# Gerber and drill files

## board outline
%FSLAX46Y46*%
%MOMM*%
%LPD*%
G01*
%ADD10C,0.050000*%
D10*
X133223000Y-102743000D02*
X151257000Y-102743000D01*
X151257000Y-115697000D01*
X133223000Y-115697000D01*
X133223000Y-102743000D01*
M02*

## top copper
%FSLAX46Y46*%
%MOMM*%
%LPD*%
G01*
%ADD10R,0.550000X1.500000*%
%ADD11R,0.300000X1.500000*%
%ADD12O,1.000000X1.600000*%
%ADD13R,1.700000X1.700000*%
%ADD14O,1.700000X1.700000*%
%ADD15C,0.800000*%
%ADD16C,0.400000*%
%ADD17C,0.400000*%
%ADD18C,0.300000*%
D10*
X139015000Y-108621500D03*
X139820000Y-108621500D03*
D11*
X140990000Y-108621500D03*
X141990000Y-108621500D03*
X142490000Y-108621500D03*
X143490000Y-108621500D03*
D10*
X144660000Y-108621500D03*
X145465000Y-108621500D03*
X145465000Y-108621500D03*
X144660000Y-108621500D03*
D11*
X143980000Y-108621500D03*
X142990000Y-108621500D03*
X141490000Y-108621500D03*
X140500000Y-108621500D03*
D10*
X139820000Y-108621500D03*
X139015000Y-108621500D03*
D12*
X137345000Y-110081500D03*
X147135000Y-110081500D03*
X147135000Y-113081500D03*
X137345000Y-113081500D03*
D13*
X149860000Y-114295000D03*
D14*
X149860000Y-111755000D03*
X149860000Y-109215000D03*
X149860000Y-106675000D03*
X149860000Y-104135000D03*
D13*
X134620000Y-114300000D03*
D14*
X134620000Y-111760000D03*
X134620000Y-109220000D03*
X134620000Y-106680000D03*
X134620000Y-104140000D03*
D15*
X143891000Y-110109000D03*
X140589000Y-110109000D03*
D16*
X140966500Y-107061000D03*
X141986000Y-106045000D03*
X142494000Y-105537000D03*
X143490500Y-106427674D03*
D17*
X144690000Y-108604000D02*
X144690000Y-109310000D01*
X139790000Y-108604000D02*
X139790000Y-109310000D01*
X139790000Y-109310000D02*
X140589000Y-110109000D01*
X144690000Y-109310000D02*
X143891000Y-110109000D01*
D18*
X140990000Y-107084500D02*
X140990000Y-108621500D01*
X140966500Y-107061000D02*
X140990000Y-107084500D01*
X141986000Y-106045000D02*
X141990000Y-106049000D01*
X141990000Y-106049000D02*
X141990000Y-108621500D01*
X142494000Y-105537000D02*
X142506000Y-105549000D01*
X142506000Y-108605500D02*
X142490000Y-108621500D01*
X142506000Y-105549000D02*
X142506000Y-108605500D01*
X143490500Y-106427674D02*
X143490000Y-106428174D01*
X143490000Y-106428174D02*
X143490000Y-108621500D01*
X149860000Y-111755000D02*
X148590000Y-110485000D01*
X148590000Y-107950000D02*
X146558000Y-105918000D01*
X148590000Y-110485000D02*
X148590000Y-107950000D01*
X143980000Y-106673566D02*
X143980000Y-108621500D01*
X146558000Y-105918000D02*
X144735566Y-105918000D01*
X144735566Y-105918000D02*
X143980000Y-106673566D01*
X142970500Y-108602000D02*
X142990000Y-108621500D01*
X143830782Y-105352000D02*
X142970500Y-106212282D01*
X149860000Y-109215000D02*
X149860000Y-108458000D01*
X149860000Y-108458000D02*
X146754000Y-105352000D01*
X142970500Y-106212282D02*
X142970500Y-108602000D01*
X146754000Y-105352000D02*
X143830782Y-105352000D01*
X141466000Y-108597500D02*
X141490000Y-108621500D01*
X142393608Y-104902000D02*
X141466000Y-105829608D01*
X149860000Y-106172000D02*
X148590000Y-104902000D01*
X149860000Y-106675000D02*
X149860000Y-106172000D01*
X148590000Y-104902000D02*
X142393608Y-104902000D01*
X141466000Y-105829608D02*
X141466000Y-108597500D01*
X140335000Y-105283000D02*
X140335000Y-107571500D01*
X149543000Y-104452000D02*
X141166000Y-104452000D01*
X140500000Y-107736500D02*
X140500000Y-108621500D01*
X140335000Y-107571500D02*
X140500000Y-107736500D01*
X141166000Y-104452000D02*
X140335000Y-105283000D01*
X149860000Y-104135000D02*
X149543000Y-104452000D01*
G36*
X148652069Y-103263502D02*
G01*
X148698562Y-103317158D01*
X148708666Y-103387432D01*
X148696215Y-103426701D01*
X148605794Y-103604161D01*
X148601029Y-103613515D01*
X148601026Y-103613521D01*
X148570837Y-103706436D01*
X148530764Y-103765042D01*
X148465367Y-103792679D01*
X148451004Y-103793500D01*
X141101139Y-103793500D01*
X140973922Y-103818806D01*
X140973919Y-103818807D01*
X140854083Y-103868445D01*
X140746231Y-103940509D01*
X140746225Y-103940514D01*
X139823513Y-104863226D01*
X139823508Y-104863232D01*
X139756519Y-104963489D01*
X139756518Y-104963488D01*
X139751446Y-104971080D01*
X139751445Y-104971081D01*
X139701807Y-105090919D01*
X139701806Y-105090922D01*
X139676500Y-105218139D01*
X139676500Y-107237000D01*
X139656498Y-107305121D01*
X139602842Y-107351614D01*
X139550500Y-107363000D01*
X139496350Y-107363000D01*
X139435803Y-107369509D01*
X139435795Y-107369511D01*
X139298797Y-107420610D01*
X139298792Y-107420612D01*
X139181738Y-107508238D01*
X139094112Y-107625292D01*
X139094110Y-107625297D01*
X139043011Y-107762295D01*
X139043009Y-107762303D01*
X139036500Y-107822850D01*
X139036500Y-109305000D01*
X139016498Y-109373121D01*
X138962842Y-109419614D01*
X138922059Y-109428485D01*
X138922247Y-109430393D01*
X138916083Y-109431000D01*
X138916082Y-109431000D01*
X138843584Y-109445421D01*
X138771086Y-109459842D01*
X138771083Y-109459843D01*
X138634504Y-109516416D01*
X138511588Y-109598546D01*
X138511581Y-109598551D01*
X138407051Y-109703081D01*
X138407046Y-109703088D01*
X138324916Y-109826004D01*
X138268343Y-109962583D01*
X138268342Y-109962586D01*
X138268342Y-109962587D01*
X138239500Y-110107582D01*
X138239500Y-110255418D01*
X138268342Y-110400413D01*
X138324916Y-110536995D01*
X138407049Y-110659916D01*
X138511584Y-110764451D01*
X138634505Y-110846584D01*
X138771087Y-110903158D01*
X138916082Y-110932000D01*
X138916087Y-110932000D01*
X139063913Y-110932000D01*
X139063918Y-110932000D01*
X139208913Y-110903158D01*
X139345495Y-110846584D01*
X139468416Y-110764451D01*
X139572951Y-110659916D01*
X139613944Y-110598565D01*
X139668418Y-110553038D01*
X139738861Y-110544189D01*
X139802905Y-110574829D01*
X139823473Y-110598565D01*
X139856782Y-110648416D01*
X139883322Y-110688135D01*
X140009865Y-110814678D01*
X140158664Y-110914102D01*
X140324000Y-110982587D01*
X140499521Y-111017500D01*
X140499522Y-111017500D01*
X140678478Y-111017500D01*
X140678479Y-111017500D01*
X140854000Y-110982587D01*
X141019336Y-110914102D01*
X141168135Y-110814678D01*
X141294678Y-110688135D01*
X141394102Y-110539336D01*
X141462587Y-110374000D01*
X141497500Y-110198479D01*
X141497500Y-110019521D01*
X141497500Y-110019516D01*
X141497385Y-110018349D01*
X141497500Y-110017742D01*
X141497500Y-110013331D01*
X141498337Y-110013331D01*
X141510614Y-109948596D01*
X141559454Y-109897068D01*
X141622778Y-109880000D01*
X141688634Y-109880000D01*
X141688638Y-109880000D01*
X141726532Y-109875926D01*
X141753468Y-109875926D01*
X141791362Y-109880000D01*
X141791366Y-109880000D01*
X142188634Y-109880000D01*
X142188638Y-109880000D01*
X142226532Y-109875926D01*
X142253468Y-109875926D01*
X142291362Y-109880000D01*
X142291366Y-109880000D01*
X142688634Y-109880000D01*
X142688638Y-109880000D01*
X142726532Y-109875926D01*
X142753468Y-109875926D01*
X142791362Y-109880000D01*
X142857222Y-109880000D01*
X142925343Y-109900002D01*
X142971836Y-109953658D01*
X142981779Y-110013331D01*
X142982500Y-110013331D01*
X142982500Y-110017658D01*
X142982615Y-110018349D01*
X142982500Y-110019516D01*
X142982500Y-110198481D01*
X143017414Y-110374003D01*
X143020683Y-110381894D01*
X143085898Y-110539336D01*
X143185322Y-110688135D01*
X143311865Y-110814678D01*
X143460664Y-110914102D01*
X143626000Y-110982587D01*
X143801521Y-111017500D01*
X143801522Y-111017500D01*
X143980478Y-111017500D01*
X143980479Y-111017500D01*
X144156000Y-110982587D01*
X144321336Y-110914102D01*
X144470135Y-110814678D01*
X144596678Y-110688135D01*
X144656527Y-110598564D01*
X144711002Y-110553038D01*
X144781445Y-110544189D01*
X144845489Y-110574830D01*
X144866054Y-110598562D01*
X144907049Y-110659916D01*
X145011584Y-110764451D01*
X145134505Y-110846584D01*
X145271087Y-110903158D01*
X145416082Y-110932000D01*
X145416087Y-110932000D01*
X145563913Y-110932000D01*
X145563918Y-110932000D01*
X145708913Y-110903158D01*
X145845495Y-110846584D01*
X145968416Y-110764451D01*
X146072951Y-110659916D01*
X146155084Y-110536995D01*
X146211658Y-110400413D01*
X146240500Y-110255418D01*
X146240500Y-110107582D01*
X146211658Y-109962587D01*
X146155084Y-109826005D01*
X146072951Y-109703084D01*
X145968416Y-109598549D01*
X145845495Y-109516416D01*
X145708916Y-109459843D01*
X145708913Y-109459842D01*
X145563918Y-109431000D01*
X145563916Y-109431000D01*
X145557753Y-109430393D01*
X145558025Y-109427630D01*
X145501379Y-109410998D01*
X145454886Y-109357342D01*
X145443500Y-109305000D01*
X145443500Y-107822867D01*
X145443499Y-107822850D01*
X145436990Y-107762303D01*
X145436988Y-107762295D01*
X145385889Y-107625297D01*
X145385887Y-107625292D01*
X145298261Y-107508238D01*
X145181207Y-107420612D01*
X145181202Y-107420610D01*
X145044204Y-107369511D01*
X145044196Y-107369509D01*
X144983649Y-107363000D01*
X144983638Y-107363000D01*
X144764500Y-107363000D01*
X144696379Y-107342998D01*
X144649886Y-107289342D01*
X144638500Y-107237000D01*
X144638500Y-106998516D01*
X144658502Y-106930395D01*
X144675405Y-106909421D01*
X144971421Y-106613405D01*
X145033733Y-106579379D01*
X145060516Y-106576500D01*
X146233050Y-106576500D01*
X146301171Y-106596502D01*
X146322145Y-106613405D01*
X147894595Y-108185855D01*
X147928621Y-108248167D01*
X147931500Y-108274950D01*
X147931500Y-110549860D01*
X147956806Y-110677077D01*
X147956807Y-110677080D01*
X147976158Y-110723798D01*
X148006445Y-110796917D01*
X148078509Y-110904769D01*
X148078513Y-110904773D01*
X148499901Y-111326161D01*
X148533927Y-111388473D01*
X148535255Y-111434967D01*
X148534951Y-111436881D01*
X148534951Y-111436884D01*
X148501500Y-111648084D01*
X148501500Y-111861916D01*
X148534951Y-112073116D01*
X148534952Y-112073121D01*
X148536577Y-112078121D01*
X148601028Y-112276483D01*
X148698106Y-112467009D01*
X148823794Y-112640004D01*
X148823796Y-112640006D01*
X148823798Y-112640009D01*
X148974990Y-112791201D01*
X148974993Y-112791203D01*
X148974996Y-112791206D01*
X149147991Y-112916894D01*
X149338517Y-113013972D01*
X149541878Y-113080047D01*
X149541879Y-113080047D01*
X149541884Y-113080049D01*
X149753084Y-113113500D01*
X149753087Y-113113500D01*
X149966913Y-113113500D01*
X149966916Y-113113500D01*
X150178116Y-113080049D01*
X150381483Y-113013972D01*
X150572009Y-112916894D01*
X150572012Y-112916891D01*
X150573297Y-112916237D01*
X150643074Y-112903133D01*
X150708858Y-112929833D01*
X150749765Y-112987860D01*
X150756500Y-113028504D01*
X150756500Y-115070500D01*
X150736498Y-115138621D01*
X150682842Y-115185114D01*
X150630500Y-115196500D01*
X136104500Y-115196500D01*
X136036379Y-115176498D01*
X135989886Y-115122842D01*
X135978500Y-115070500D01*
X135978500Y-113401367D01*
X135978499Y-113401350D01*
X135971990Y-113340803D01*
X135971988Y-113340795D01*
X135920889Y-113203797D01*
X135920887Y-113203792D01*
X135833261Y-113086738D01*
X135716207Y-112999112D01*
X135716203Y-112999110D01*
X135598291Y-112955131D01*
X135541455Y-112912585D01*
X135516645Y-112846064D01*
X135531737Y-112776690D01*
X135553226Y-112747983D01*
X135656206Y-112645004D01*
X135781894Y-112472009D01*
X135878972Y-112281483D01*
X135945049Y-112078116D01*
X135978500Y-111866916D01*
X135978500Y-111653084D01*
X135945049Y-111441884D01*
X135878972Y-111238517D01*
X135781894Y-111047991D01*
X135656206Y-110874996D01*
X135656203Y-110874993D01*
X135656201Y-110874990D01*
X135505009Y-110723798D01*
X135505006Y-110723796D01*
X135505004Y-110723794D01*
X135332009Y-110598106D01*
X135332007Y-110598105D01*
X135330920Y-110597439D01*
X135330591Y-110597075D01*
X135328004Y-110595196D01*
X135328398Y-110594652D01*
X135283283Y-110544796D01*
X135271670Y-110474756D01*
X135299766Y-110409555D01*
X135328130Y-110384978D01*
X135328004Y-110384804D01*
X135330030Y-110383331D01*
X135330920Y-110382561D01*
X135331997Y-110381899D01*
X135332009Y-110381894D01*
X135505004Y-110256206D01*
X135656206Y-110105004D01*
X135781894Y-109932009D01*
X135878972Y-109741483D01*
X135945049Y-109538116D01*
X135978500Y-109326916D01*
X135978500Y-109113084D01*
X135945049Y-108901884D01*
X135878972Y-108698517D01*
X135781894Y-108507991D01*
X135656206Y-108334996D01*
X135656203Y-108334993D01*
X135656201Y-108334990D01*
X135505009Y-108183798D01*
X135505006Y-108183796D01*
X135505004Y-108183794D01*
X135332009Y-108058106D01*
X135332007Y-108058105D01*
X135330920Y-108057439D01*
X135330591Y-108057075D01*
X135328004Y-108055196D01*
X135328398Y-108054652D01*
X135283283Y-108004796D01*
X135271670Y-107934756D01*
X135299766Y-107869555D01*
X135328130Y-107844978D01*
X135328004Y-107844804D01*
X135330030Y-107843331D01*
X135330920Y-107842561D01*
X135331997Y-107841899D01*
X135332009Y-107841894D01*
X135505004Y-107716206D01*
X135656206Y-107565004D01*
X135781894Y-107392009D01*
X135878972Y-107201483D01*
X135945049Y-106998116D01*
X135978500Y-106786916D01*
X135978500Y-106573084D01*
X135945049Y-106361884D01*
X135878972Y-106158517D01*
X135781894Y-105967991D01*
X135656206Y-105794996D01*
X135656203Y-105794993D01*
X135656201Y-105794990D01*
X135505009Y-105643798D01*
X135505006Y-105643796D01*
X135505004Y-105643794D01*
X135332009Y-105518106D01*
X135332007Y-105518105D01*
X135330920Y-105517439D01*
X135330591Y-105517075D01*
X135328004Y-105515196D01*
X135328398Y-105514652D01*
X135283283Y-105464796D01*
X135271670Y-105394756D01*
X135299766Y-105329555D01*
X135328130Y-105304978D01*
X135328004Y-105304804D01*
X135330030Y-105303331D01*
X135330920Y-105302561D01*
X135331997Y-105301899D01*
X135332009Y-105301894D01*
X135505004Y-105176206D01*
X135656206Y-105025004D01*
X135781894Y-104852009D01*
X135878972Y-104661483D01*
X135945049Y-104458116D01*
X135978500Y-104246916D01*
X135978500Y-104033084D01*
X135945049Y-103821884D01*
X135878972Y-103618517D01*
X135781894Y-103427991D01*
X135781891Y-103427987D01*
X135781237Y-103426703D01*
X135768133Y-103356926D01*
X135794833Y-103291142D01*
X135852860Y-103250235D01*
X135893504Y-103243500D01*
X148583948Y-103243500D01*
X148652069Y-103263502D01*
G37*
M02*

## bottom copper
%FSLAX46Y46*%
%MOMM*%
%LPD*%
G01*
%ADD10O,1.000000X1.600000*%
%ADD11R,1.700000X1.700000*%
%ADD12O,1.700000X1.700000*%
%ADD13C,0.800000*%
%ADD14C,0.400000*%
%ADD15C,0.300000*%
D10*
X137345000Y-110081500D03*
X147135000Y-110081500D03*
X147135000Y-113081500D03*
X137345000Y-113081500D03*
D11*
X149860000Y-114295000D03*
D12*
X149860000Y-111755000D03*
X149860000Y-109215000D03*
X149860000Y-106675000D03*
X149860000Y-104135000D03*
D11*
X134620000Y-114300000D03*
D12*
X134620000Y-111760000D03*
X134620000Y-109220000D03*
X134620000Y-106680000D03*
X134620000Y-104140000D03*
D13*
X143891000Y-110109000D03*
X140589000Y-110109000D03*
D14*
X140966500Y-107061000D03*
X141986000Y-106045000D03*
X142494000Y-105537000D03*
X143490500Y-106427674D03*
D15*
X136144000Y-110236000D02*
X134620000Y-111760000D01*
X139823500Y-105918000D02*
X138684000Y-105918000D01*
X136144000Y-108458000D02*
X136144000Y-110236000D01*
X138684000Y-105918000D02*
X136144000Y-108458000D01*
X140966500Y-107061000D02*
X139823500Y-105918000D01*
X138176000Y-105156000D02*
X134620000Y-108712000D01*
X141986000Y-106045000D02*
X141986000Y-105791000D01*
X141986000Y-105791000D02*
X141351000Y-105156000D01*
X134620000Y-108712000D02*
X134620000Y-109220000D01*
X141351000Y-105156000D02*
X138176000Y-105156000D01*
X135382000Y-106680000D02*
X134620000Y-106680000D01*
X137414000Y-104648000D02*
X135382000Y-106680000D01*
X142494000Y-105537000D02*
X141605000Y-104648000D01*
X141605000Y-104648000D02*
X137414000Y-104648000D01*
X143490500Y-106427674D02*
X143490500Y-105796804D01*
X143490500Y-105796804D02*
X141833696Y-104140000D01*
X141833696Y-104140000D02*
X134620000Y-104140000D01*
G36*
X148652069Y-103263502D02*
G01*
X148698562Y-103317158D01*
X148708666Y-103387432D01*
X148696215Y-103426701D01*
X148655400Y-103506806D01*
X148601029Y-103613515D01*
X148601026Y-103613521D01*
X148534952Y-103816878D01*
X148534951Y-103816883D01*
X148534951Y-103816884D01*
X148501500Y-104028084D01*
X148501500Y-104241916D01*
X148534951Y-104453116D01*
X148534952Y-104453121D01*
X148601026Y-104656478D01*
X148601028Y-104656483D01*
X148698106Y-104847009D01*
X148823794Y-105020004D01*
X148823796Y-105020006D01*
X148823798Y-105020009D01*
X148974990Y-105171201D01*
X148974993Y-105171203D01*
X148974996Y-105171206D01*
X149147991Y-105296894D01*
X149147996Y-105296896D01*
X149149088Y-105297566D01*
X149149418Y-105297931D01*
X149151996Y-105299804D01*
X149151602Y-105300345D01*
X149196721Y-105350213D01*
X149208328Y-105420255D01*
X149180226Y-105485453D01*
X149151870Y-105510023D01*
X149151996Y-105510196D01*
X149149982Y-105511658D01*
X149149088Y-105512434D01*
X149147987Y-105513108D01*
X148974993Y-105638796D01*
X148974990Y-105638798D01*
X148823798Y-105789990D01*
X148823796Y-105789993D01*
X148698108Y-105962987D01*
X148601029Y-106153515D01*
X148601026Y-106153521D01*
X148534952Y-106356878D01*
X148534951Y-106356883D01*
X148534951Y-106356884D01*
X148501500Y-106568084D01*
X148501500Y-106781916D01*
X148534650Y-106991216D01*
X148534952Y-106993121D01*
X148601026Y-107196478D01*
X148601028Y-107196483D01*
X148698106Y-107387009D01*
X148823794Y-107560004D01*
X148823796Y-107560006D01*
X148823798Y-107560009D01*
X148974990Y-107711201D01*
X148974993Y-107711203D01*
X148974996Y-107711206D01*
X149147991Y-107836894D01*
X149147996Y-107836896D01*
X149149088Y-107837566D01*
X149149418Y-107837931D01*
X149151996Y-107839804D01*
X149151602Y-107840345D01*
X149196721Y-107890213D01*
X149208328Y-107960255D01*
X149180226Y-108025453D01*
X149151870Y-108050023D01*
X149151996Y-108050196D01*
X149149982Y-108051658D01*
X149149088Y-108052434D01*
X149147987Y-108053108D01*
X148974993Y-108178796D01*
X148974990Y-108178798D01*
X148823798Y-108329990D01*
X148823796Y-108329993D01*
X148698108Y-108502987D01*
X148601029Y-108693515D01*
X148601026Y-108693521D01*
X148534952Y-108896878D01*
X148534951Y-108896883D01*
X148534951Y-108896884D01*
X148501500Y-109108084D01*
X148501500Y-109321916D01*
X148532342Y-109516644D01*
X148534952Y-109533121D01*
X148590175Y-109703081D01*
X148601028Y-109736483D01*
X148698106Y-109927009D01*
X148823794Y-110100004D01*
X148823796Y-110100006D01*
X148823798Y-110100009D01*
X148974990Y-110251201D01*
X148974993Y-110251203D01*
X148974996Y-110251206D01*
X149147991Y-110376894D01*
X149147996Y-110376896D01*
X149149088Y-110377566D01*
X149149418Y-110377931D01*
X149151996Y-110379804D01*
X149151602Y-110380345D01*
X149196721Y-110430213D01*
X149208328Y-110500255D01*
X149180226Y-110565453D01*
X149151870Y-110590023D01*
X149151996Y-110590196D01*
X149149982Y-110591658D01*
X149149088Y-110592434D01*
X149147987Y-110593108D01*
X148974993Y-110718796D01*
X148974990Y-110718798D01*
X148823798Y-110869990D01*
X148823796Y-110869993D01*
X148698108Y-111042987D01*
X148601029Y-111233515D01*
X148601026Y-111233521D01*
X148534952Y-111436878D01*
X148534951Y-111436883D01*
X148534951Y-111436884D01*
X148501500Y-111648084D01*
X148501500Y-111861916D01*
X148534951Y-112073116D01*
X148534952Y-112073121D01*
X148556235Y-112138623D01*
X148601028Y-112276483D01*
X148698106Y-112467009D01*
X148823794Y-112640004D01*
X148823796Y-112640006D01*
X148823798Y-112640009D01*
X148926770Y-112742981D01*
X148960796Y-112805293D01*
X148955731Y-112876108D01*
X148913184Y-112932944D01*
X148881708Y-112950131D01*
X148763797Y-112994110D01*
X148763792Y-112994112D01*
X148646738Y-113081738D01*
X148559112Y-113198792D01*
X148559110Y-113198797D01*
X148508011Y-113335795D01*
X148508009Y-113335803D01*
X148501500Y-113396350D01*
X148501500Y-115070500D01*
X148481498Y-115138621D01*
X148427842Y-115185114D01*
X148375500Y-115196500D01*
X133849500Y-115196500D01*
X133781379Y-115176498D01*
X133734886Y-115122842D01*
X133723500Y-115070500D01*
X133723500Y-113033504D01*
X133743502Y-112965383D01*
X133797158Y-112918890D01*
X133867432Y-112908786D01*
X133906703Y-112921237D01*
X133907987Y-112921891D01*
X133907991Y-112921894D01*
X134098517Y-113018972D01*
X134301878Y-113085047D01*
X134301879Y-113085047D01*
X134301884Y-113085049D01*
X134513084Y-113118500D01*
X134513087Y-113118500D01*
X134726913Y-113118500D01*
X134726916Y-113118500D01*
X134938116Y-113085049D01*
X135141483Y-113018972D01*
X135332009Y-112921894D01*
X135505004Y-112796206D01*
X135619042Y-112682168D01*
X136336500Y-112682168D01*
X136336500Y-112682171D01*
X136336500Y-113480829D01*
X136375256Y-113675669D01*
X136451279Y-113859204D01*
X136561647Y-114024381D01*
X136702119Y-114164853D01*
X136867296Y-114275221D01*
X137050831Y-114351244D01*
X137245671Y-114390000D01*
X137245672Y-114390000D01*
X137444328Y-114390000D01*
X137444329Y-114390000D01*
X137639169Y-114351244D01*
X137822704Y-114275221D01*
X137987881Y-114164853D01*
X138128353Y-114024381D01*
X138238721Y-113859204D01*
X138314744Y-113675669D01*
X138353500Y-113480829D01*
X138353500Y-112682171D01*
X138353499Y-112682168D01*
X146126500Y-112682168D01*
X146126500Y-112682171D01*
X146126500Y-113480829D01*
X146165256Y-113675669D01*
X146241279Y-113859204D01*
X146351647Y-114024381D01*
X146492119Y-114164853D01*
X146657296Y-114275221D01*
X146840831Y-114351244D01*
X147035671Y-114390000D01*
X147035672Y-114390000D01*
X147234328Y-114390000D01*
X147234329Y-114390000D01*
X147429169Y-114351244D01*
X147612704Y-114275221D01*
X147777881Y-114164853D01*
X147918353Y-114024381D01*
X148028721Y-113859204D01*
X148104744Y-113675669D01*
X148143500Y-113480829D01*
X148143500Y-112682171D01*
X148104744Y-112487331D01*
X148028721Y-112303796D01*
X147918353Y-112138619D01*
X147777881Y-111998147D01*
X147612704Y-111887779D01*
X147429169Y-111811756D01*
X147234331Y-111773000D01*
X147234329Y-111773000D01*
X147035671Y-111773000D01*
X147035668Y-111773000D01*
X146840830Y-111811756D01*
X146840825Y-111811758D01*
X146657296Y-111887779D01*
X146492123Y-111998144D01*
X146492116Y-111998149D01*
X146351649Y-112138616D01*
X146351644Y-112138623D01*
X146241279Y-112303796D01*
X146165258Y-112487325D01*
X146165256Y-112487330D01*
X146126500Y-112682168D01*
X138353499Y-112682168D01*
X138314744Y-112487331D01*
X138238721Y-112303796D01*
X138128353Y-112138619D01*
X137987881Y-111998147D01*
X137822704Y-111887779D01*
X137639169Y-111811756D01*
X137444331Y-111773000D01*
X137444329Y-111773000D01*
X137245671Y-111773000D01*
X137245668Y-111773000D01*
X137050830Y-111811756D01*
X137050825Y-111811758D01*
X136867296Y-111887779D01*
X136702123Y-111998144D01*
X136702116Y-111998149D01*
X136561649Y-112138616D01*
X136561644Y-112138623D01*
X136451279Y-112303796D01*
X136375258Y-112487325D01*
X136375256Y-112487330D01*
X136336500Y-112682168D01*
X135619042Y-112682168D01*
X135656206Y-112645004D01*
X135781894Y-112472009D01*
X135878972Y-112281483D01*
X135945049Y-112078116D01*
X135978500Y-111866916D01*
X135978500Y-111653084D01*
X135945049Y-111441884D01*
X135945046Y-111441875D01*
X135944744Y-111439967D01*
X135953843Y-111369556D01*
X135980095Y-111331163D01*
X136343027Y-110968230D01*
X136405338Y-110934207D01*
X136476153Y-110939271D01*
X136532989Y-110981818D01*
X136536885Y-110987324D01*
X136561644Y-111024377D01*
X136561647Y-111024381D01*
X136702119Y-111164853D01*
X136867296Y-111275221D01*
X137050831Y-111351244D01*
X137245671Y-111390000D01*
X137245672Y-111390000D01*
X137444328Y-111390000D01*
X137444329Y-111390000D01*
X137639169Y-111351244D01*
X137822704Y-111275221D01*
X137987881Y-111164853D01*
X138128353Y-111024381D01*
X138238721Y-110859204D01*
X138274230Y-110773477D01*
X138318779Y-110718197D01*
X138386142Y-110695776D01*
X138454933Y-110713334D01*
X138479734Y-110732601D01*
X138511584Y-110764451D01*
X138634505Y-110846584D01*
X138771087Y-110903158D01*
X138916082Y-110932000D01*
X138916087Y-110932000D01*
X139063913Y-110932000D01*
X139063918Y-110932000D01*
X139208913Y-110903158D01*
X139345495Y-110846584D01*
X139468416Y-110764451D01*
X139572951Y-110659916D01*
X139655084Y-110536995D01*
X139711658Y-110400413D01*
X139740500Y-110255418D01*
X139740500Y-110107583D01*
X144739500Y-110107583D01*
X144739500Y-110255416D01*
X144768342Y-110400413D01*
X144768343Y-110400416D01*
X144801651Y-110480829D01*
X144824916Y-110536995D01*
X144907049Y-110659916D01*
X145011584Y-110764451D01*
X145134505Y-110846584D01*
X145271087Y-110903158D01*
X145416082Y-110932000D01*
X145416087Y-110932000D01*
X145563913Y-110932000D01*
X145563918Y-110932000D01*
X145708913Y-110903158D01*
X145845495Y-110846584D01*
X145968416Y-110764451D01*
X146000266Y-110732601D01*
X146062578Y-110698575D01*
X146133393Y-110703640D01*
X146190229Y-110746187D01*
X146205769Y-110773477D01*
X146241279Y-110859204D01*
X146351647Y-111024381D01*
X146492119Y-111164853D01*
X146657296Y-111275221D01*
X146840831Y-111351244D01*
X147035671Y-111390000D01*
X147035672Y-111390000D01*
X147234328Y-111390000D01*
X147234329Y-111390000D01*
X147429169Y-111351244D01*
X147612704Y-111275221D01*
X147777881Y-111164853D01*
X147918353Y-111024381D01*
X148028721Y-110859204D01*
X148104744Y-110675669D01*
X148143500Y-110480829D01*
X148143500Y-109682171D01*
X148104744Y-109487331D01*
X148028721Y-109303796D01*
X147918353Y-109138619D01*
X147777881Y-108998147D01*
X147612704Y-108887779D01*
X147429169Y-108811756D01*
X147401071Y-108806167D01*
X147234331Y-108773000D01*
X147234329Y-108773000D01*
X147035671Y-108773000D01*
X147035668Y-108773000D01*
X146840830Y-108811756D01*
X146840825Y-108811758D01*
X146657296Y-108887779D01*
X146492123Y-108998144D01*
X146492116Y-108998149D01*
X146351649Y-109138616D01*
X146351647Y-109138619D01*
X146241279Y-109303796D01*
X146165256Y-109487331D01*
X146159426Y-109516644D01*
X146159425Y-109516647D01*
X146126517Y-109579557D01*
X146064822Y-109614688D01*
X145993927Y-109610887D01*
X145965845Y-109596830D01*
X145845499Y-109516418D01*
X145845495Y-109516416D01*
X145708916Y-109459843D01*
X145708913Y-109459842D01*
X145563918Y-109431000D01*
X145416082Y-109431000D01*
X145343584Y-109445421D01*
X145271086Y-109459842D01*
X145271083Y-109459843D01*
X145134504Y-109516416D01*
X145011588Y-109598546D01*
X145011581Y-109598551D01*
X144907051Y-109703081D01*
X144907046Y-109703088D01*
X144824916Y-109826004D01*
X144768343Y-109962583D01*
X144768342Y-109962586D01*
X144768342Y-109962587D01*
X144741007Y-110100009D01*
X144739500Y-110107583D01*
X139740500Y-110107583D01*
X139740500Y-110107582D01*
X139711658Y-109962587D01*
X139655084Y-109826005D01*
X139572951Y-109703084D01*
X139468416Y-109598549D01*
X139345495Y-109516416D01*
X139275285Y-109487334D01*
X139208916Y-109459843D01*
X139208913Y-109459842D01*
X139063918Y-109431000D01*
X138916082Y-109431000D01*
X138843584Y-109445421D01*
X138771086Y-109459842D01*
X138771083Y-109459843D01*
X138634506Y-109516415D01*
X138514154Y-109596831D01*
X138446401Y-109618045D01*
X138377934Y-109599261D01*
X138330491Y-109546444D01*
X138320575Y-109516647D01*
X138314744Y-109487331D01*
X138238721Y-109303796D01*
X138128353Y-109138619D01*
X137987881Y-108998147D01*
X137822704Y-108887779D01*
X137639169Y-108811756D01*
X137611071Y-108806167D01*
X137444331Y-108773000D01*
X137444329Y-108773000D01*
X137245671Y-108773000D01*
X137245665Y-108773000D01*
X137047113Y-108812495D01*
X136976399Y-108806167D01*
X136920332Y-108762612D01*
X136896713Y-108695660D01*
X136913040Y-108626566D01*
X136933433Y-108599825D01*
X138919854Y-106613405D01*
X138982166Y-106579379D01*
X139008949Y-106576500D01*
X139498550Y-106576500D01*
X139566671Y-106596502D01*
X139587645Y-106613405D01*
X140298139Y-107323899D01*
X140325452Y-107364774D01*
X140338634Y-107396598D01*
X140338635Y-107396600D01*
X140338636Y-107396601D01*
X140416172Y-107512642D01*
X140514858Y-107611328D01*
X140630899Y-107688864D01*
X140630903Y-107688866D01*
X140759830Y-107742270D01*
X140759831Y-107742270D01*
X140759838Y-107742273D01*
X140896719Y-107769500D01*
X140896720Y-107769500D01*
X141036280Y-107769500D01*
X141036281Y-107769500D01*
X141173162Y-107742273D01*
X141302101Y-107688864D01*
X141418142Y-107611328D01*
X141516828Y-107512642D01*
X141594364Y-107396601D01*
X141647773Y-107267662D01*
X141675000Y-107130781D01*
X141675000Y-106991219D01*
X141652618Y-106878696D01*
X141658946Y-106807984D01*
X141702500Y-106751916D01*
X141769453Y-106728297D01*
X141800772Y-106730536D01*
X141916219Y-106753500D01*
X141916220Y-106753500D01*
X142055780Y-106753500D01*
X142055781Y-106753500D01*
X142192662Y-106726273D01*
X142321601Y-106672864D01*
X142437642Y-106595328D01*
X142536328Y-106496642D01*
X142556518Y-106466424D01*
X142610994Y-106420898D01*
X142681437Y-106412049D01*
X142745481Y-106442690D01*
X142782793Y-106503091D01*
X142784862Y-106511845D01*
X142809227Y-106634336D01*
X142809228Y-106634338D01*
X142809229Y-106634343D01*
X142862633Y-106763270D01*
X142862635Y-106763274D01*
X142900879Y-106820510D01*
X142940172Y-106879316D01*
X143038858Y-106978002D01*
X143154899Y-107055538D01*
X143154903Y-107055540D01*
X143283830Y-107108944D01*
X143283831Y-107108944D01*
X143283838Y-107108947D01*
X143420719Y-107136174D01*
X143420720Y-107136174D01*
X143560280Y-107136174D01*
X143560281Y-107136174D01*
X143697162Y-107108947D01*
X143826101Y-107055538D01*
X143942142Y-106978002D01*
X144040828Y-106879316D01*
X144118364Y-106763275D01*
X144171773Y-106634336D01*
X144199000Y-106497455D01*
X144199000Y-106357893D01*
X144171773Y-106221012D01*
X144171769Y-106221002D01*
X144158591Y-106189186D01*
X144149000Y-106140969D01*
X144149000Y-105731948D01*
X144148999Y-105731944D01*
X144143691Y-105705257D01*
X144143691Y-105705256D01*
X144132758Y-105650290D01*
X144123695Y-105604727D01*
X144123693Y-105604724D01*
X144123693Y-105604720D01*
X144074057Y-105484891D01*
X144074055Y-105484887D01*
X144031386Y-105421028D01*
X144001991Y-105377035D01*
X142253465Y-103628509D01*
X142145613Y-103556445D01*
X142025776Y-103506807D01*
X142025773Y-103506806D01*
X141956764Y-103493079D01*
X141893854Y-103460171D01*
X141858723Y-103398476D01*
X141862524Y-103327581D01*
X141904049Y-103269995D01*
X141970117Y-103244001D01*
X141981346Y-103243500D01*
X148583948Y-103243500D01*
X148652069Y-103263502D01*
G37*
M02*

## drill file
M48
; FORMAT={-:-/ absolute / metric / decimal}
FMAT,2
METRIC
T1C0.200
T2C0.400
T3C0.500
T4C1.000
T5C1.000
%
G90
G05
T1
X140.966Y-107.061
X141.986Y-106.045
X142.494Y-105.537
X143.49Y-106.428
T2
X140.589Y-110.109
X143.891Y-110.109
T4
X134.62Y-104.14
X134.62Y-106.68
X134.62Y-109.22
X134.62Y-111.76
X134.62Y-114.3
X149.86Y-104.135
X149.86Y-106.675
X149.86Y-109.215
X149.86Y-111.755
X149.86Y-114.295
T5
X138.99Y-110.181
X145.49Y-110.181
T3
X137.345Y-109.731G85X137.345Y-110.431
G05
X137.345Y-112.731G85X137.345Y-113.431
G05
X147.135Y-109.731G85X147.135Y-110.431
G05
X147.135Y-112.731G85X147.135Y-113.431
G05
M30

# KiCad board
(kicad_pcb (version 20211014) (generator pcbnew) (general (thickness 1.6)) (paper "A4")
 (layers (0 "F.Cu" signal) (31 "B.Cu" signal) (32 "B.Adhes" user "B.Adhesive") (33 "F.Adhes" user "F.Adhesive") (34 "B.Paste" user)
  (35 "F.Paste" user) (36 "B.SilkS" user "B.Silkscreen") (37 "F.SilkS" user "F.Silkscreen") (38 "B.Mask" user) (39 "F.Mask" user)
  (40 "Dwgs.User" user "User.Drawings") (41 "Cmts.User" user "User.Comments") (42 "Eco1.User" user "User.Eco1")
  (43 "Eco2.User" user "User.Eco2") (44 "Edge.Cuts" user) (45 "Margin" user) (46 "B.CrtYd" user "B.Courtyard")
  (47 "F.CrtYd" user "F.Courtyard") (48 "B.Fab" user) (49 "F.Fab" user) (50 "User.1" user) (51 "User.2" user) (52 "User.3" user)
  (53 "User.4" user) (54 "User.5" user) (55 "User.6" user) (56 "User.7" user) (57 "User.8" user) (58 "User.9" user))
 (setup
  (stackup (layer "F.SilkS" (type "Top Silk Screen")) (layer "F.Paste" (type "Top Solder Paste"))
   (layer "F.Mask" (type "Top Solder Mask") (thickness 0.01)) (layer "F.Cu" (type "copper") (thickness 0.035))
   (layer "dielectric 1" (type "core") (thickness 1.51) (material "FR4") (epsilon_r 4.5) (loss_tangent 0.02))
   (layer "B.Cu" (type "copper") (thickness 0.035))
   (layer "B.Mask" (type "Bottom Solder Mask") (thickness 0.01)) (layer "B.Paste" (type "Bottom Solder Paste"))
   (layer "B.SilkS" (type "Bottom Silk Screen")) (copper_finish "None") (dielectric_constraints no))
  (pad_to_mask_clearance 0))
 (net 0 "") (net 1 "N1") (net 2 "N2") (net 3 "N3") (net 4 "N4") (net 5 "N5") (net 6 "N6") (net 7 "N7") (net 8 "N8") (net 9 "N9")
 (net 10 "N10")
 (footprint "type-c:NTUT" (layer "F.Cu") (at 142.621 104.648 180)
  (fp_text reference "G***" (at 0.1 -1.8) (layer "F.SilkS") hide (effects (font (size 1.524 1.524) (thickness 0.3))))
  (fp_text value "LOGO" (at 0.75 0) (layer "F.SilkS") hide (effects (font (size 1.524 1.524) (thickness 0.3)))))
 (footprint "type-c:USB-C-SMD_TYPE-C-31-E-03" (layer "F.Cu") (at 142.24 110.8515)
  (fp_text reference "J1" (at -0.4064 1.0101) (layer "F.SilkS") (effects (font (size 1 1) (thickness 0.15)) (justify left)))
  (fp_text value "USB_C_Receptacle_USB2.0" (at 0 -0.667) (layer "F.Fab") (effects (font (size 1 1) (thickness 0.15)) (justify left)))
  (pad "" np_thru_hole circle (at 3.25 -0.67) (size 1 1) (drill 1) (layers *.Cu *.Mask))
  (pad "" np_thru_hole circle (at -3.25 -0.67) (size 1 1) (drill 1) (layers *.Cu *.Mask))
  (pad "A1" smd rect (at -3.225 -2.23) (size 0.55 1.5) (layers "F.Cu" "F.Paste" "F.Mask") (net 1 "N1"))
  (pad "A4" smd rect (at -2.42 -2.23) (size 0.55 1.5) (layers "F.Cu" "F.Paste" "F.Mask") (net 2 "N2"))
  (pad "A5" smd rect (at -1.25 -2.23) (size 0.3 1.5) (layers "F.Cu" "F.Paste" "F.Mask") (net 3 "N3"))
  (pad "A6" smd rect (at -0.25 -2.23) (size 0.3 1.5) (layers "F.Cu" "F.Paste" "F.Mask") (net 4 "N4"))
  (pad "A7" smd rect (at 0.25 -2.23) (size 0.3 1.5) (layers "F.Cu" "F.Paste" "F.Mask") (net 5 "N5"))
  (pad "A8" smd rect (at 1.25 -2.23) (size 0.3 1.5) (layers "F.Cu" "F.Paste" "F.Mask") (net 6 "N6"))
  (pad "A9" smd rect (at 2.42 -2.23) (size 0.55 1.5) (layers "F.Cu" "F.Paste" "F.Mask") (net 2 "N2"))
  (pad "A12" smd rect (at 3.225 -2.23) (size 0.55 1.5) (layers "F.Cu" "F.Paste" "F.Mask") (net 1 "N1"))
  (pad "B1" smd rect (at 3.225 -2.23) (size 0.55 1.5) (layers "F.Cu" "F.Paste" "F.Mask") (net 1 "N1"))
  (pad "B4" smd rect (at 2.42 -2.23) (size 0.55 1.5) (layers "F.Cu" "F.Paste" "F.Mask") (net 2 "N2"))
  (pad "B5" smd rect (at 1.74 -2.23) (size 0.3 1.5) (layers "F.Cu" "F.Paste" "F.Mask") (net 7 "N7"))
  (pad "B6" smd rect (at 0.75 -2.23) (size 0.3 1.5) (layers "F.Cu" "F.Paste" "F.Mask") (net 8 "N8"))
  (pad "B7" smd rect (at -0.75 -2.23) (size 0.3 1.5) (layers "F.Cu" "F.Paste" "F.Mask") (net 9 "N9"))
  (pad "B8" smd rect (at -1.74 -2.23) (size 0.3 1.5) (layers "F.Cu" "F.Paste" "F.Mask") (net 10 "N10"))
  (pad "B9" smd rect (at -2.42 -2.23) (size 0.55 1.5) (layers "F.Cu" "F.Paste" "F.Mask") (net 2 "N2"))
  (pad "B12" smd rect (at -3.225 -2.23) (size 0.55 1.5) (layers "F.Cu" "F.Paste" "F.Mask") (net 1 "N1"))
  (pad "S1" thru_hole oval (at -4.895 -0.77) (size 1 1.6) (drill oval 0.5 1.2) (layers *.Cu *.Mask) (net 1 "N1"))
  (pad "S1" thru_hole oval (at 4.895 -0.77) (size 1 1.6) (drill oval 0.5 1.2) (layers *.Cu *.Mask) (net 1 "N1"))
  (pad "S1" thru_hole oval (at 4.895 2.23) (size 1 1.6) (drill oval 0.5 1.2) (layers *.Cu *.Mask) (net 1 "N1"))
  (pad "S1" thru_hole oval (at -4.895 2.23) (size 1 1.6) (drill oval 0.5 1.2) (layers *.Cu *.Mask) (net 1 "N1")))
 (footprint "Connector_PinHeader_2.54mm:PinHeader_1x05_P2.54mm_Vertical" (layer "B.Cu") (at 149.86 114.295)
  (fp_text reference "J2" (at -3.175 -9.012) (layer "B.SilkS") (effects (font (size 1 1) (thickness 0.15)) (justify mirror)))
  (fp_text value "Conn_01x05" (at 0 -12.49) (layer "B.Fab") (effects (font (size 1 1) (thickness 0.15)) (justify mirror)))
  (pad "1" thru_hole rect (at 0 0) (size 1.7 1.7) (drill 1) (layers *.Cu *.Mask) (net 1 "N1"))
  (pad "2" thru_hole oval (at 0 -2.54) (size 1.7 1.7) (drill 1) (layers *.Cu *.Mask) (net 7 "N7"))
  (pad "3" thru_hole oval (at 0 -5.08) (size 1.7 1.7) (drill 1) (layers *.Cu *.Mask) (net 8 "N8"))
  (pad "4" thru_hole oval (at 0 -7.62) (size 1.7 1.7) (drill 1) (layers *.Cu *.Mask) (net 9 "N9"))
  (pad "5" thru_hole oval (at 0 -10.16) (size 1.7 1.7) (drill 1) (layers *.Cu *.Mask) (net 10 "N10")))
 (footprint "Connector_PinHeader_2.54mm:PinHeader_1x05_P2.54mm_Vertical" (layer "B.Cu") (at 134.62 114.3)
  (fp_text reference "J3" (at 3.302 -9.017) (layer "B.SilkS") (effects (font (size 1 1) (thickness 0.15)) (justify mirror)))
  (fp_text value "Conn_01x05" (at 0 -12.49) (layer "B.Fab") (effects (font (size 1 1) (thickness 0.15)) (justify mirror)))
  (pad "1" thru_hole rect (at 0 0) (size 1.7 1.7) (drill 1) (layers *.Cu *.Mask) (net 2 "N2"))
  (pad "2" thru_hole oval (at 0 -2.54) (size 1.7 1.7) (drill 1) (layers *.Cu *.Mask) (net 3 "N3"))
  (pad "3" thru_hole oval (at 0 -5.08) (size 1.7 1.7) (drill 1) (layers *.Cu *.Mask) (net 4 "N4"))
  (pad "4" thru_hole oval (at 0 -7.62) (size 1.7 1.7) (drill 1) (layers *.Cu *.Mask) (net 5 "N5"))
  (pad "5" thru_hole oval (at 0 -10.16) (size 1.7 1.7) (drill 1) (layers *.Cu *.Mask) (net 6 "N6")))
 (gr_rect (start 133.223 102.743) (end 151.257 115.697) (layer "Edge.Cuts") (width 0.05) (fill none))
 (segment (start 144.69 108.604) (end 144.69 109.31) (width 0.4) (layer "F.Cu") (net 2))
 (segment (start 139.79 108.604) (end 139.79 109.31) (width 0.4) (layer "F.Cu") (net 2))
 (segment (start 139.79 109.31) (end 140.589 110.109) (width 0.4) (layer "F.Cu") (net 2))
 (segment (start 144.69 109.31) (end 143.891 110.109) (width 0.4) (layer "F.Cu") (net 2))
 (via (at 143.891 110.109) (size 0.8) (drill 0.4) (layers "F.Cu" "B.Cu") (free) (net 2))
 (via (at 140.589 110.109) (size 0.8) (drill 0.4) (layers "F.Cu" "B.Cu") (free) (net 2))
 (segment (start 140.99 107.0845) (end 140.99 108.6215) (width 0.3) (layer "F.Cu") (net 3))
 (segment (start 140.9665 107.061) (end 140.99 107.0845) (width 0.3) (layer "F.Cu") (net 3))
 (via (at 140.9665 107.061) (size 0.4) (drill 0.2) (layers "F.Cu" "B.Cu") (free) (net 3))
 (segment (start 136.144 110.236) (end 134.62 111.76) (width 0.3) (layer "B.Cu") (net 3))
 (segment (start 139.8235 105.918) (end 138.684 105.918) (width 0.3) (layer "B.Cu") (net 3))
 (segment (start 136.144 108.458) (end 136.144 110.236) (width 0.3) (layer "B.Cu") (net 3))
 (segment (start 138.684 105.918) (end 136.144 108.458) (width 0.3) (layer "B.Cu") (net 3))
 (segment (start 140.9665 107.061) (end 139.8235 105.918) (width 0.3) (layer "B.Cu") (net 3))
 (segment (start 141.986 106.045) (end 141.99 106.049) (width 0.3) (layer "F.Cu") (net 4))
 (segment (start 141.99 106.049) (end 141.99 108.6215) (width 0.3) (layer "F.Cu") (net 4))
 (via (at 141.986 106.045) (size 0.4) (drill 0.2) (layers "F.Cu" "B.Cu") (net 4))
 (segment (start 138.176 105.156) (end 134.62 108.712) (width 0.3) (layer "B.Cu") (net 4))
 (segment (start 141.986 106.045) (end 141.986 105.791) (width 0.3) (layer "B.Cu") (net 4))
 (segment (start 141.986 105.791) (end 141.351 105.156) (width 0.3) (layer "B.Cu") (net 4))
 (segment (start 134.62 108.712) (end 134.62 109.22) (width 0.3) (layer "B.Cu") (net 4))
 (segment (start 141.351 105.156) (end 138.176 105.156) (width 0.3) (layer "B.Cu") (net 4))
 (segment (start 142.494 105.537) (end 142.506 105.549) (width 0.3) (layer "F.Cu") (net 5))
 (segment (start 142.506 108.6055) (end 142.49 108.6215) (width 0.3) (layer "F.Cu") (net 5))
 (segment (start 142.506 105.549) (end 142.506 108.6055) (width 0.3) (layer "F.Cu") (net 5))
 (via (at 142.494 105.537) (size 0.4) (drill 0.2) (layers "F.Cu" "B.Cu") (free) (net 5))
 (segment (start 135.382 106.68) (end 134.62 106.68) (width 0.3) (layer "B.Cu") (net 5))
 (segment (start 137.414 104.648) (end 135.382 106.68) (width 0.3) (layer "B.Cu") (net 5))
 (segment (start 142.494 105.537) (end 141.605 104.648) (width 0.3) (layer "B.Cu") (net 5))
 (segment (start 141.605 104.648) (end 137.414 104.648) (width 0.3) (layer "B.Cu") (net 5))
 (segment (start 143.4905 106.427674) (end 143.49 106.428174) (width 0.3) (layer "F.Cu") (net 6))
 (segment (start 143.49 106.428174) (end 143.49 108.6215) (width 0.3) (layer "F.Cu") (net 6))
 (via (at 143.4905 106.427674) (size 0.4) (drill 0.2) (layers "F.Cu" "B.Cu") (free) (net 6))
 (segment (start 143.4905 106.427674) (end 143.4905 105.796804) (width 0.3) (layer "B.Cu") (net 6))
 (segment (start 143.4905 105.796804) (end 141.833696 104.14) (width 0.3) (layer "B.Cu") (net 6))
 (segment (start 141.833696 104.14) (end 134.62 104.14) (width 0.3) (layer "B.Cu") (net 6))
 (segment (start 149.86 111.755) (end 148.59 110.485) (width 0.3) (layer "F.Cu") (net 7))
 (segment (start 148.59 107.95) (end 146.558 105.918) (width 0.3) (layer "F.Cu") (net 7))
 (segment (start 148.59 110.485) (end 148.59 107.95) (width 0.3) (layer "F.Cu") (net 7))
 (segment (start 143.98 106.673566) (end 143.98 108.6215) (width 0.3) (layer "F.Cu") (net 7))
 (segment (start 146.558 105.918) (end 144.735566 105.918) (width 0.3) (layer "F.Cu") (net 7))
 (segment (start 144.735566 105.918) (end 143.98 106.673566) (width 0.3) (layer "F.Cu") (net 7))
 (segment (start 142.9705 108.602) (end 142.99 108.6215) (width 0.3) (layer "F.Cu") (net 8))
 (segment (start 143.830782 105.352) (end 142.9705 106.212282) (width 0.3) (layer "F.Cu") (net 8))
 (segment (start 149.86 109.215) (end 149.86 108.458) (width 0.3) (layer "F.Cu") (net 8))
 (segment (start 149.86 108.458) (end 146.754 105.352) (width 0.3) (layer "F.Cu") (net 8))
 (segment (start 142.9705 106.212282) (end 142.9705 108.602) (width 0.3) (layer "F.Cu") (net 8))
 (segment (start 146.754 105.352) (end 143.830782 105.352) (width 0.3) (layer "F.Cu") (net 8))
 (segment (start 141.466 108.5975) (end 141.49 108.6215) (width 0.3) (layer "F.Cu") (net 9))
 (segment (start 142.393608 104.902) (end 141.466 105.829608) (width 0.3) (layer "F.Cu") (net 9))
 (segment (start 149.86 106.172) (end 148.59 104.902) (width 0.3) (layer "F.Cu") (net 9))
 (segment (start 149.86 106.675) (end 149.86 106.172) (width 0.3) (layer "F.Cu") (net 9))
 (segment (start 148.59 104.902) (end 142.393608 104.902) (width 0.3) (layer "F.Cu") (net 9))
 (segment (start 141.466 105.829608) (end 141.466 108.5975) (width 0.3) (layer "F.Cu") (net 9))
 (segment (start 140.335 105.283) (end 140.335 107.5715) (width 0.3) (layer "F.Cu") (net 10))
 (segment (start 149.543 104.452) (end 141.166 104.452) (width 0.3) (layer "F.Cu") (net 10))
 (segment (start 140.5 107.7365) (end 140.5 108.6215) (width 0.3) (layer "F.Cu") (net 10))
 (segment (start 140.335 107.5715) (end 140.5 107.7365) (width 0.3) (layer "F.Cu") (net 10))
 (segment (start 141.166 104.452) (end 140.335 105.283) (width 0.3) (layer "F.Cu") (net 10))
 (segment (start 149.86 104.135) (end 149.543 104.452) (width 0.3) (layer "F.Cu") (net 10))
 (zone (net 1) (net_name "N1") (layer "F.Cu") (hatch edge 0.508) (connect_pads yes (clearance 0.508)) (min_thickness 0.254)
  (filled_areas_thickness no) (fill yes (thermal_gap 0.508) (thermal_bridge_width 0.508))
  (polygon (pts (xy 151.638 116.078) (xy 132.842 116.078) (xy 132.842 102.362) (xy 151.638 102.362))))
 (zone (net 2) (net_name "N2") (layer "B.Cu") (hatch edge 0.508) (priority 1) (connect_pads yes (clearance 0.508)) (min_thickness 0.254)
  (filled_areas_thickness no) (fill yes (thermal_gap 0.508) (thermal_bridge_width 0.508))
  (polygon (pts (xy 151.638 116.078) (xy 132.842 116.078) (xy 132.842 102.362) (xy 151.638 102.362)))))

